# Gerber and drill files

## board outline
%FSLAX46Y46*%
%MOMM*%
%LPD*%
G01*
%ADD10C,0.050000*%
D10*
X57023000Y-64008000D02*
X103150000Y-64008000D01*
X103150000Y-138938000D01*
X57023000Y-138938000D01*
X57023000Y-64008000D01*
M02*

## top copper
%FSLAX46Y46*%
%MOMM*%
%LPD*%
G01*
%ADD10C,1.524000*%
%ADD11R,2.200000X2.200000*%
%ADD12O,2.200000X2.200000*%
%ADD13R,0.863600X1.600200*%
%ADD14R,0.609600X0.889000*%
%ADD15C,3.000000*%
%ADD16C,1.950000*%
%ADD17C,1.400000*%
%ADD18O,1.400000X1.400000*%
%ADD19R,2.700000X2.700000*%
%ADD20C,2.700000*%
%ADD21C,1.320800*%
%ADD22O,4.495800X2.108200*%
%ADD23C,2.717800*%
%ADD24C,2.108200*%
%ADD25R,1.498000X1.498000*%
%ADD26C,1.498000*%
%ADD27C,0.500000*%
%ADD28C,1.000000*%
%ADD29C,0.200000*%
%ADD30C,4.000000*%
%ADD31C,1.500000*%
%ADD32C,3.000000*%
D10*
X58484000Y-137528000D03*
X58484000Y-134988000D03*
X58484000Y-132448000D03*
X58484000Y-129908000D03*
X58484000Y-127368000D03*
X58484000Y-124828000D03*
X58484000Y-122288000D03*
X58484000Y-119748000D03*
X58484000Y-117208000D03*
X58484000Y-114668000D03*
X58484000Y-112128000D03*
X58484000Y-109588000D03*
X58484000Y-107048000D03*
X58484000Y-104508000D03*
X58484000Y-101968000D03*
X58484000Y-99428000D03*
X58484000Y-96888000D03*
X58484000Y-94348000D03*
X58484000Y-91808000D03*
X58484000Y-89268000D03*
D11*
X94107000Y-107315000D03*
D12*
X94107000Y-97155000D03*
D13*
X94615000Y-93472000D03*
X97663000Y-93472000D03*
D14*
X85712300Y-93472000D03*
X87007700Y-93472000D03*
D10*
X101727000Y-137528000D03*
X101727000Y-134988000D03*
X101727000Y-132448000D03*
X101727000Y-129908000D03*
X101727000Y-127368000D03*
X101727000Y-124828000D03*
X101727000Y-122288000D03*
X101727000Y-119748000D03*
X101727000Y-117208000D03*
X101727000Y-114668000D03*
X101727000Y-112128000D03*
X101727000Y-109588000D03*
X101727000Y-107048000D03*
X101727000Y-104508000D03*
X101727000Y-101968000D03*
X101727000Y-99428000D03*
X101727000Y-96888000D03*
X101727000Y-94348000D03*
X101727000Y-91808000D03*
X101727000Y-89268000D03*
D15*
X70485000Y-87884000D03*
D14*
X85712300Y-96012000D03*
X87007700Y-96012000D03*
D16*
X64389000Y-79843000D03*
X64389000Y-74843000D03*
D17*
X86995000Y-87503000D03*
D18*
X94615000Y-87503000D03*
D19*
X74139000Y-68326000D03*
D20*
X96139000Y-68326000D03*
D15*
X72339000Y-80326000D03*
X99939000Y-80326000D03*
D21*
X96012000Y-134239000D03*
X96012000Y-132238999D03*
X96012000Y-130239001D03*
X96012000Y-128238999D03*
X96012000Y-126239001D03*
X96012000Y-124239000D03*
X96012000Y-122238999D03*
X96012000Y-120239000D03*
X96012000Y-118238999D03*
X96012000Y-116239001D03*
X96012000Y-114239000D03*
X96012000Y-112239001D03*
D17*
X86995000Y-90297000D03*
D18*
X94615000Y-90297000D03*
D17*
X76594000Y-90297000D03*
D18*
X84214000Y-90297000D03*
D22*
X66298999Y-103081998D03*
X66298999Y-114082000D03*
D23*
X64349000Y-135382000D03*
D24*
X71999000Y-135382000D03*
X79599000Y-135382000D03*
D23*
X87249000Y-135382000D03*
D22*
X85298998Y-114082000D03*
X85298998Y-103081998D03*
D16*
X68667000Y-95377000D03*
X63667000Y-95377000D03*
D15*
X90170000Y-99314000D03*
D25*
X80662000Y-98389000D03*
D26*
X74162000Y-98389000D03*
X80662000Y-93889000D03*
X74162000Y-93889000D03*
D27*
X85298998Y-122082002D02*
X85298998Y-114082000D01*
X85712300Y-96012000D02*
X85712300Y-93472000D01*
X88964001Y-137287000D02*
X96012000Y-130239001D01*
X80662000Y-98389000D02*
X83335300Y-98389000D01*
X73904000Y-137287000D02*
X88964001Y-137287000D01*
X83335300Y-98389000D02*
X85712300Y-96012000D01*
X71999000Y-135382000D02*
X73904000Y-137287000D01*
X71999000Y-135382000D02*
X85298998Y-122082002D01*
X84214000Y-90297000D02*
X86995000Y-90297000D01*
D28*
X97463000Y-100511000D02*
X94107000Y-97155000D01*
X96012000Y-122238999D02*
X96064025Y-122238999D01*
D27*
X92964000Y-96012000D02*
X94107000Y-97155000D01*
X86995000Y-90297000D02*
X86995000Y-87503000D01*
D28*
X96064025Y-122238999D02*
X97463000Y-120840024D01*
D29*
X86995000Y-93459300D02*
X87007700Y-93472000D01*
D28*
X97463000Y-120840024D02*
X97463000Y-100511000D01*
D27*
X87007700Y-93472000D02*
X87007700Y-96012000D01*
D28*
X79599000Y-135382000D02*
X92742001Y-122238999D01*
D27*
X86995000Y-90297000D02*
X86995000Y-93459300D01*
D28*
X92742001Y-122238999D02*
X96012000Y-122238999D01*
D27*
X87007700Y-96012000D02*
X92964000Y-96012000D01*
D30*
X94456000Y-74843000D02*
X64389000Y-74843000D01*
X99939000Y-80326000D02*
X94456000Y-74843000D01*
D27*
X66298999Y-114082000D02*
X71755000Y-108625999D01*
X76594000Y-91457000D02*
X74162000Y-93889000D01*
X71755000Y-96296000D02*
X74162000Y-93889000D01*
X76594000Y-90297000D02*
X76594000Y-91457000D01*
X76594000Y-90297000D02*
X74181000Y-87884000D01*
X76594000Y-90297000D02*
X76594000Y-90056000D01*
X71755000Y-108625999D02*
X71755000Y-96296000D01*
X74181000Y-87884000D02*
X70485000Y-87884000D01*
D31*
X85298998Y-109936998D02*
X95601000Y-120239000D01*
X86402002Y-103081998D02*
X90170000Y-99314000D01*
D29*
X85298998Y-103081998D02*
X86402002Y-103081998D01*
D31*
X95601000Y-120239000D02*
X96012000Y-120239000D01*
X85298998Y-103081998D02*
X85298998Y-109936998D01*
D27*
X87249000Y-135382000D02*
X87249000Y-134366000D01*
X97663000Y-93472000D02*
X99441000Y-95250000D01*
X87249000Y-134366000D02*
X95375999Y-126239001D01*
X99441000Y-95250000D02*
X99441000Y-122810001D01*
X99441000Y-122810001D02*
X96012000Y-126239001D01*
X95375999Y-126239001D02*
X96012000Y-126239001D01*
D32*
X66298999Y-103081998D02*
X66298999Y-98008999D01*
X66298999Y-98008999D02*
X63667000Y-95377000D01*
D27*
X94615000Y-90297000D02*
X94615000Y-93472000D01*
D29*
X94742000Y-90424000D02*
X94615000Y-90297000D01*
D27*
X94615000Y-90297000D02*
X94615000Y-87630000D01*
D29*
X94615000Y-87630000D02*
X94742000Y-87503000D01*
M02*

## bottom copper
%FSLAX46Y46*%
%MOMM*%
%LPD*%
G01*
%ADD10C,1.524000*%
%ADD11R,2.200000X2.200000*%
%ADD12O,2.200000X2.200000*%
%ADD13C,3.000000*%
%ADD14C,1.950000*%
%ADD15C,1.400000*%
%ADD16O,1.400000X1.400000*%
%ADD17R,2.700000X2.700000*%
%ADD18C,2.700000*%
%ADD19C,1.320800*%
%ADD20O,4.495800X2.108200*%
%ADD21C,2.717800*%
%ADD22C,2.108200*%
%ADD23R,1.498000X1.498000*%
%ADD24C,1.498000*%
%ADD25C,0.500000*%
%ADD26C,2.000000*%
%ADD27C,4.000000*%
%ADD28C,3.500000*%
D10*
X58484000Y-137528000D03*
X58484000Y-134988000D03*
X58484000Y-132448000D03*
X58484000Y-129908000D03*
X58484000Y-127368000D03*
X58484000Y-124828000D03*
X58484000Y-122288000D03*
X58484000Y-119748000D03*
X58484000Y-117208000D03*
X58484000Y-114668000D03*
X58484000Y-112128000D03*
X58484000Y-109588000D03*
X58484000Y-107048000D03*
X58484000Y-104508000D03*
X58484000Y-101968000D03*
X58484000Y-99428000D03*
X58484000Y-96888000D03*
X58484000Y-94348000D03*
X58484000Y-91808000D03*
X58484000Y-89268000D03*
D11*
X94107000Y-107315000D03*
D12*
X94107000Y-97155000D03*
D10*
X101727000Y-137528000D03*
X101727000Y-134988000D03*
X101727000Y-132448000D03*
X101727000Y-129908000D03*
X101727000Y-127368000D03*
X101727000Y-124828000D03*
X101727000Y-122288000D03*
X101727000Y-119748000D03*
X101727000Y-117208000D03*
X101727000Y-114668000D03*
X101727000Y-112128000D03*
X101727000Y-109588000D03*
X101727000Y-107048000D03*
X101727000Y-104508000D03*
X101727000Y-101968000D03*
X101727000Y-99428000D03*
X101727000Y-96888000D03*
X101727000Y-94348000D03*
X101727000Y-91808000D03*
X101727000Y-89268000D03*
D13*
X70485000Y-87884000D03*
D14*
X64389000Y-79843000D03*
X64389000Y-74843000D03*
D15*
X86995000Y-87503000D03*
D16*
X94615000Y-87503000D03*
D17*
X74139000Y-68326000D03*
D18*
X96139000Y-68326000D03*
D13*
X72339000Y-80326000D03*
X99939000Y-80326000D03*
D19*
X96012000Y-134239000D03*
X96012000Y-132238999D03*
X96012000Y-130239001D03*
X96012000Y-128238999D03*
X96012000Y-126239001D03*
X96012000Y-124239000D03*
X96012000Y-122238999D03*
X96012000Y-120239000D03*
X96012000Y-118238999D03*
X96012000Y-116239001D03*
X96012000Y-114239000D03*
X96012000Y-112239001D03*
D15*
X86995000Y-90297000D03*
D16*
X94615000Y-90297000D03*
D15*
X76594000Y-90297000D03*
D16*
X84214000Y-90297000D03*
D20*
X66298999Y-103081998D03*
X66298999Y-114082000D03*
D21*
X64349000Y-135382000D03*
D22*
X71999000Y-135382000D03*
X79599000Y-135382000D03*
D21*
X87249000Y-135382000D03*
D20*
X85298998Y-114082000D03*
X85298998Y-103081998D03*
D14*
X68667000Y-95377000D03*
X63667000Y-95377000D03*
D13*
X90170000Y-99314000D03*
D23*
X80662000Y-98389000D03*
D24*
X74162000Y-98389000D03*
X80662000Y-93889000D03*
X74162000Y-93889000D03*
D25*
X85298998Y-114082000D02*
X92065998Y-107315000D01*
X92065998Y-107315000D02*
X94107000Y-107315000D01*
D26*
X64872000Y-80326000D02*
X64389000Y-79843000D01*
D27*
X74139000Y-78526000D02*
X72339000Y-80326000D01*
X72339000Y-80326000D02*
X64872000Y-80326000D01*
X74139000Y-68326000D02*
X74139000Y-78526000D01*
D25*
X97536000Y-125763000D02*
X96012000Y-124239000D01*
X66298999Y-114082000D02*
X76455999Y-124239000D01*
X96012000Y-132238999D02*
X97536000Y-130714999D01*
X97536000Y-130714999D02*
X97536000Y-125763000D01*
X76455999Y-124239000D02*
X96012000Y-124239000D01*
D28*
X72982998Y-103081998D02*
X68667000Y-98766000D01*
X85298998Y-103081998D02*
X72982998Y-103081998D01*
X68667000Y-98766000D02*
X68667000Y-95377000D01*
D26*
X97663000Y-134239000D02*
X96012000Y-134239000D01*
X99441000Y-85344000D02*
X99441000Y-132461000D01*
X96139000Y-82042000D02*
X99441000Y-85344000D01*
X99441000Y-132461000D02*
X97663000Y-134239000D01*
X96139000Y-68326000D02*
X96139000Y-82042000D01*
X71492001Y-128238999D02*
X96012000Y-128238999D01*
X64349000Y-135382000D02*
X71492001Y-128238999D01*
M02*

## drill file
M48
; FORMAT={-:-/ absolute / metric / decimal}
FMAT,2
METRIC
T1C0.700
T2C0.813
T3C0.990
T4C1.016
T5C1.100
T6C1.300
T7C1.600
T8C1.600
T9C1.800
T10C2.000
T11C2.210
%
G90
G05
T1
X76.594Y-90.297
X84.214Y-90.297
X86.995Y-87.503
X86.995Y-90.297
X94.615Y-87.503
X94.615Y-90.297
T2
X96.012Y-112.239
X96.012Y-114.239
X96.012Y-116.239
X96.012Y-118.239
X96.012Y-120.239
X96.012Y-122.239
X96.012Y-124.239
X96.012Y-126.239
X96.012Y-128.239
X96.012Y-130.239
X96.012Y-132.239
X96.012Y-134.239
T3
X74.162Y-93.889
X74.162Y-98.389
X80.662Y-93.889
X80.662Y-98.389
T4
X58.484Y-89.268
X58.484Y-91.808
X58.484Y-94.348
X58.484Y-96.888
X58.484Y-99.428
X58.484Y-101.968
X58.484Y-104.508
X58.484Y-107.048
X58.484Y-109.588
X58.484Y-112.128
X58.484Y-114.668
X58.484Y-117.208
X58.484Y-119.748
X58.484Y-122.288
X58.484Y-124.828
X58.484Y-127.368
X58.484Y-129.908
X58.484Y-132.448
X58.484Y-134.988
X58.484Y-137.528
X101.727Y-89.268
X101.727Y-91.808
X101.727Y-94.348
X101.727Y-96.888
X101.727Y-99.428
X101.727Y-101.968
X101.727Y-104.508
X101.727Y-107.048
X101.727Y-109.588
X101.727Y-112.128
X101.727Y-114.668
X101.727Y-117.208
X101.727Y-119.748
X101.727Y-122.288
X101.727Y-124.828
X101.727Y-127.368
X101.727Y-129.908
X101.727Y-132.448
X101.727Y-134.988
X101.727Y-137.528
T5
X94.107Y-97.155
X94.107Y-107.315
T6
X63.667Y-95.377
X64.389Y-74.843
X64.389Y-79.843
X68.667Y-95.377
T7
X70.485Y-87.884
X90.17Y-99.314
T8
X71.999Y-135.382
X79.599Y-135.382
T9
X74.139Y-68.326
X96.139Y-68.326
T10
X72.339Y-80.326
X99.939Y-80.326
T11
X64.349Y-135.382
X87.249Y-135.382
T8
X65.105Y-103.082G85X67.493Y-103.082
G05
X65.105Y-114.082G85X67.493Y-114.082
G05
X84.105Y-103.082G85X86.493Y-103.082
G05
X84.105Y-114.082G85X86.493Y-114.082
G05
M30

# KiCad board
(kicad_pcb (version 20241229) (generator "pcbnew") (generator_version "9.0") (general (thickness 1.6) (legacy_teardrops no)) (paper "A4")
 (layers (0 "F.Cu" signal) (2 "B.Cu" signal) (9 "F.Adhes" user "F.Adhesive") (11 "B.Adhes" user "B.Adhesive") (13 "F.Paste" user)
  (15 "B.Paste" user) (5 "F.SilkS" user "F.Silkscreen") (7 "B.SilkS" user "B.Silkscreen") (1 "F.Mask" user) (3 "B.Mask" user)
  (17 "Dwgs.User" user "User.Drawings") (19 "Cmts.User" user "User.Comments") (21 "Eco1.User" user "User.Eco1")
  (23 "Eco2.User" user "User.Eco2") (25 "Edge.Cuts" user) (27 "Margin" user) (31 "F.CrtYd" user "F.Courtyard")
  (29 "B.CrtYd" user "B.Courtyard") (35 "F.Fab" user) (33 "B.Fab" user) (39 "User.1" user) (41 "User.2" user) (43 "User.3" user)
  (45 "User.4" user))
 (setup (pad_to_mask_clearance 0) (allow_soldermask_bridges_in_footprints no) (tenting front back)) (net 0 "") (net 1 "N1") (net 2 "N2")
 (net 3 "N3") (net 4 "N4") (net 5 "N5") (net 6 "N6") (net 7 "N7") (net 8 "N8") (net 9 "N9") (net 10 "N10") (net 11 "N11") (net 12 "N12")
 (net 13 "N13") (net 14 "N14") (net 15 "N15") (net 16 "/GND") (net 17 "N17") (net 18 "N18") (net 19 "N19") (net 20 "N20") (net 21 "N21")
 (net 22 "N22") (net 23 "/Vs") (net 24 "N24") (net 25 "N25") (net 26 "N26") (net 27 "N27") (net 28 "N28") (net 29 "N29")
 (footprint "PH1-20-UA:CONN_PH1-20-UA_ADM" (layer "F.Cu") (at 58.484 137.528 90)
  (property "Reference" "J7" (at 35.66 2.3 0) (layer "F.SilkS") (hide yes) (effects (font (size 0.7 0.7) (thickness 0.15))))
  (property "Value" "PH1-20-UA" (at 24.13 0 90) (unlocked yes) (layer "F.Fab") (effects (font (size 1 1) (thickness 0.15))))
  (pad "1" thru_hole circle (at 0 0 90) (size 1.524 1.524) (drill 1.016) (layers "*.Cu" "*.Mask") (remove_unused_layers no))
  (pad "2" thru_hole circle (at 2.54 0 90) (size 1.524 1.524) (drill 1.016) (layers "*.Cu" "*.Mask") (remove_unused_layers no))
  (pad "3" thru_hole circle (at 5.08 0 90) (size 1.524 1.524) (drill 1.016) (layers "*.Cu" "*.Mask") (remove_unused_layers no))
  (pad "4" thru_hole circle (at 7.62 0 90) (size 1.524 1.524) (drill 1.016) (layers "*.Cu" "*.Mask") (remove_unused_layers no))
  (pad "5" thru_hole circle (at 10.16 0 90) (size 1.524 1.524) (drill 1.016) (layers "*.Cu" "*.Mask") (remove_unused_layers no))
  (pad "6" thru_hole circle (at 12.7 0 90) (size 1.524 1.524) (drill 1.016) (layers "*.Cu" "*.Mask") (remove_unused_layers no))
  (pad "7" thru_hole circle (at 15.24 0 90) (size 1.524 1.524) (drill 1.016) (layers "*.Cu" "*.Mask") (remove_unused_layers no) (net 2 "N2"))
  (pad "8" thru_hole circle (at 17.78 0 90) (size 1.524 1.524) (drill 1.016) (layers "*.Cu" "*.Mask") (remove_unused_layers no) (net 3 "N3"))
  (pad "9" thru_hole circle (at 20.32 0 90) (size 1.524 1.524) (drill 1.016) (layers "*.Cu" "*.Mask") (remove_unused_layers no) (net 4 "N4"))
  (pad "10" thru_hole circle (at 22.86 0 90) (size 1.524 1.524) (drill 1.016) (layers "*.Cu" "*.Mask") (remove_unused_layers no)
   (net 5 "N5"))
  (pad "11" thru_hole circle (at 25.4 0 90) (size 1.524 1.524) (drill 1.016) (layers "*.Cu" "*.Mask") (remove_unused_layers no) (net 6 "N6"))
  (pad "12" thru_hole circle (at 27.94 0 90) (size 1.524 1.524) (drill 1.016) (layers "*.Cu" "*.Mask") (remove_unused_layers no)
   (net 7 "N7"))
  (pad "13" thru_hole circle (at 30.48 0 90) (size 1.524 1.524) (drill 1.016) (layers "*.Cu" "*.Mask") (remove_unused_layers no)
   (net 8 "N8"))
  (pad "14" thru_hole circle (at 33.02 0 90) (size 1.524 1.524) (drill 1.016) (layers "*.Cu" "*.Mask") (remove_unused_layers no)
   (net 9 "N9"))
  (pad "15" thru_hole circle (at 35.56 0 90) (size 1.524 1.524) (drill 1.016) (layers "*.Cu" "*.Mask") (remove_unused_layers no)
   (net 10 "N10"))
  (pad "16" thru_hole circle (at 38.1 0 90) (size 1.524 1.524) (drill 1.016) (layers "*.Cu" "*.Mask") (remove_unused_layers no)
   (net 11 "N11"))
  (pad "17" thru_hole circle (at 40.64 0 90) (size 1.524 1.524) (drill 1.016) (layers "*.Cu" "*.Mask") (remove_unused_layers no)
   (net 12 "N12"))
  (pad "18" thru_hole circle (at 43.18 0 90) (size 1.524 1.524) (drill 1.016) (layers "*.Cu" "*.Mask") (remove_unused_layers no)
   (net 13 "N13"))
  (pad "19" thru_hole circle (at 45.72 0 90) (size 1.524 1.524) (drill 1.016) (layers "*.Cu" "*.Mask") (remove_unused_layers no)
   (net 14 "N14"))
  (pad "20" thru_hole circle (at 48.26 0 90) (size 1.524 1.524) (drill 1.016) (layers "*.Cu" "*.Mask") (remove_unused_layers no)
   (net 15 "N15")))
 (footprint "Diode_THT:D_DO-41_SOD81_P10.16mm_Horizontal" (layer "F.Cu") (at 94.107 107.315 90)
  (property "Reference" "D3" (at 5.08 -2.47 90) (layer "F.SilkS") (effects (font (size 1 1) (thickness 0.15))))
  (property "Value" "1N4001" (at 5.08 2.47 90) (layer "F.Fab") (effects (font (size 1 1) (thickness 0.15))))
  (pad "1" thru_hole rect (at 0 0 90) (size 2.2 2.2) (drill 1.1) (layers "*.Cu" "*.Mask") (remove_unused_layers no) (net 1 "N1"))
  (pad "2" thru_hole oval (at 10.16 0 90) (size 2.2 2.2) (drill 1.1) (layers "*.Cu" "*.Mask") (remove_unused_layers no) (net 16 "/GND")))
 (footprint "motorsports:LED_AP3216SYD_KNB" (layer "F.Cu") (at 96.139 93.472)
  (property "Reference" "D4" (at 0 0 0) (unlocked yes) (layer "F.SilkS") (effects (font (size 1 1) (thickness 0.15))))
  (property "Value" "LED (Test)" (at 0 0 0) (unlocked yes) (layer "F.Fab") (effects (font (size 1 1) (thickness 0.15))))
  (pad "1" smd rect (at -1.524 0) (size 0.8636 1.6002) (layers "F.Cu" "F.Mask" "F.Paste") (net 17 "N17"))
  (pad "2" smd rect (at 1.524 0) (size 0.8636 1.6002) (layers "F.Cu" "F.Mask" "F.Paste") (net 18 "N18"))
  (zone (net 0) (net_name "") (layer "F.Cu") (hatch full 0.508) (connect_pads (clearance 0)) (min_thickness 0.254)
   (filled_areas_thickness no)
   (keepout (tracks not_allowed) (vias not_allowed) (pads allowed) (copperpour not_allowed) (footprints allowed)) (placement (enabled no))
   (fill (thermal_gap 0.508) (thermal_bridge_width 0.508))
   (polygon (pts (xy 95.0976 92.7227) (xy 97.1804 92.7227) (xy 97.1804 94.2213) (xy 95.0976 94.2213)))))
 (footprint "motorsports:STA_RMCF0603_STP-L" (layer "F.Cu") (at 86.36 93.472)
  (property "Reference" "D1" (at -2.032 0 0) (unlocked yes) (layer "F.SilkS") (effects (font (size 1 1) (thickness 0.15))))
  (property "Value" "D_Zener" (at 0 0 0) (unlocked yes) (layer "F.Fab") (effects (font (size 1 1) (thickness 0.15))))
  (pad "1" smd rect (at -0.6477 0) (size 0.6096 0.889) (layers "F.Cu" "F.Mask" "F.Paste") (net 1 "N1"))
  (pad "2" smd rect (at 0.6477 0) (size 0.6096 0.889) (layers "F.Cu" "F.Mask" "F.Paste") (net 16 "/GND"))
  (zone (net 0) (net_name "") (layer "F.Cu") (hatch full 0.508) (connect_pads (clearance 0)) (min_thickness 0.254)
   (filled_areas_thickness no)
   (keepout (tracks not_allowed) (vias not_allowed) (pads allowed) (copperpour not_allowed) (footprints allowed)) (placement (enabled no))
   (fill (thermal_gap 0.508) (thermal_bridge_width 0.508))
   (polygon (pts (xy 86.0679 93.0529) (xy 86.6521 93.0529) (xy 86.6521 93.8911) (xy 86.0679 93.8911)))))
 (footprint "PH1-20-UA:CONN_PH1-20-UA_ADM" (layer "F.Cu") (at 101.727 137.528 90)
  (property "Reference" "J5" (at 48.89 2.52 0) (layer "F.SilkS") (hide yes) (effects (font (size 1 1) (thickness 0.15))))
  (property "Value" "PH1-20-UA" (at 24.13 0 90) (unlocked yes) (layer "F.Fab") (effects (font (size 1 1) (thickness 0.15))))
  (pad "1" thru_hole circle (at 0 0 90) (size 1.524 1.524) (drill 1.016) (layers "*.Cu" "*.Mask") (remove_unused_layers no))
  (pad "2" thru_hole circle (at 2.54 0 90) (size 1.524 1.524) (drill 1.016) (layers "*.Cu" "*.Mask") (remove_unused_layers no))
  (pad "3" thru_hole circle (at 5.08 0 90) (size 1.524 1.524) (drill 1.016) (layers "*.Cu" "*.Mask") (remove_unused_layers no))
  (pad "4" thru_hole circle (at 7.62 0 90) (size 1.524 1.524) (drill 1.016) (layers "*.Cu" "*.Mask") (remove_unused_layers no))
  (pad "5" thru_hole circle (at 10.16 0 90) (size 1.524 1.524) (drill 1.016) (layers "*.Cu" "*.Mask") (remove_unused_layers no))
  (pad "6" thru_hole circle (at 12.7 0 90) (size 1.524 1.524) (drill 1.016) (layers "*.Cu" "*.Mask") (remove_unused_layers no))
  (pad "7" thru_hole circle (at 15.24 0 90) (size 1.524 1.524) (drill 1.016) (layers "*.Cu" "*.Mask") (remove_unused_layers no))
  (pad "8" thru_hole circle (at 17.78 0 90) (size 1.524 1.524) (drill 1.016) (layers "*.Cu" "*.Mask") (remove_unused_layers no))
  (pad "9" thru_hole circle (at 20.32 0 90) (size 1.524 1.524) (drill 1.016) (layers "*.Cu" "*.Mask") (remove_unused_layers no))
  (pad "10" thru_hole circle (at 22.86 0 90) (size 1.524 1.524) (drill 1.016) (layers "*.Cu" "*.Mask") (remove_unused_layers no))
  (pad "11" thru_hole circle (at 25.4 0 90) (size 1.524 1.524) (drill 1.016) (layers "*.Cu" "*.Mask") (remove_unused_layers no))
  (pad "12" thru_hole circle (at 27.94 0 90) (size 1.524 1.524) (drill 1.016) (layers "*.Cu" "*.Mask") (remove_unused_layers no))
  (pad "13" thru_hole circle (at 30.48 0 90) (size 1.524 1.524) (drill 1.016) (layers "*.Cu" "*.Mask") (remove_unused_layers no))
  (pad "14" thru_hole circle (at 33.02 0 90) (size 1.524 1.524) (drill 1.016) (layers "*.Cu" "*.Mask") (remove_unused_layers no))
  (pad "15" thru_hole circle (at 35.56 0 90) (size 1.524 1.524) (drill 1.016) (layers "*.Cu" "*.Mask") (remove_unused_layers no))
  (pad "16" thru_hole circle (at 38.1 0 90) (size 1.524 1.524) (drill 1.016) (layers "*.Cu" "*.Mask") (remove_unused_layers no))
  (pad "17" thru_hole circle (at 40.64 0 90) (size 1.524 1.524) (drill 1.016) (layers "*.Cu" "*.Mask") (remove_unused_layers no))
  (pad "18" thru_hole circle (at 43.18 0 90) (size 1.524 1.524) (drill 1.016) (layers "*.Cu" "*.Mask") (remove_unused_layers no))
  (pad "19" thru_hole circle (at 45.72 0 90) (size 1.524 1.524) (drill 1.016) (layers "*.Cu" "*.Mask") (remove_unused_layers no))
  (pad "20" thru_hole circle (at 48.26 0 90) (size 1.524 1.524) (drill 1.016) (layers "*.Cu" "*.Mask") (remove_unused_layers no)))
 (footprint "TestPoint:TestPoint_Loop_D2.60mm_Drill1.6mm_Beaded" (layer "F.Cu") (at 70.485 87.884)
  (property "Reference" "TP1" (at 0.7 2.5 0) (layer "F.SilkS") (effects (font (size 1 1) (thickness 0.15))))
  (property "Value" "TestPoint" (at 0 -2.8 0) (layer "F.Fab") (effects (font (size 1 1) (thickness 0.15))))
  (pad "1" thru_hole circle (at 0 0) (size 3 3) (drill 1.6) (layers "*.Cu" "*.Mask") (remove_unused_layers no) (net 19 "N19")))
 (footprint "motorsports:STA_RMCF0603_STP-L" (layer "F.Cu") (at 86.36 96.012)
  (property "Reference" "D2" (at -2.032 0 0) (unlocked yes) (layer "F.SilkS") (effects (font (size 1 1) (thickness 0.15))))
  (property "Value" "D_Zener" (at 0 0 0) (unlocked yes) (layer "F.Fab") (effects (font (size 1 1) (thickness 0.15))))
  (pad "1" smd rect (at -0.6477 0) (size 0.6096 0.889) (layers "F.Cu" "F.Mask" "F.Paste") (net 1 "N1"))
  (pad "2" smd rect (at 0.6477 0) (size 0.6096 0.889) (layers "F.Cu" "F.Mask" "F.Paste") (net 16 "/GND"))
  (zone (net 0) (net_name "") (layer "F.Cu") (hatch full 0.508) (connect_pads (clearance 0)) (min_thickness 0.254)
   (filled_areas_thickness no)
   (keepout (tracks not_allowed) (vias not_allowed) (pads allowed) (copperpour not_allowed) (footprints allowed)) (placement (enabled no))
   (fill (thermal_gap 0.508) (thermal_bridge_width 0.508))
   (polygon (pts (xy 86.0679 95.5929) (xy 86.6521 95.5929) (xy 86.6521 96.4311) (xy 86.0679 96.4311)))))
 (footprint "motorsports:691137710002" (layer "F.Cu") (at 64.389 77.343 90)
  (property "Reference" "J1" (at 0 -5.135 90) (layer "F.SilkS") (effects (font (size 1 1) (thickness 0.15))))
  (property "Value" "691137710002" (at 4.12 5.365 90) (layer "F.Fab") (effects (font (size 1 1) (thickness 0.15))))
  (pad "1" thru_hole circle (at -2.5 0 90) (size 1.95 1.95) (drill 1.3) (layers "*.Cu" "*.Mask") (remove_unused_layers no) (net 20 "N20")
   (solder_mask_margin 0.102))
  (pad "2" thru_hole circle (at 2.5 0 90) (size 1.95 1.95) (drill 1.3) (layers "*.Cu" "*.Mask") (remove_unused_layers no) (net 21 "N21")
   (solder_mask_margin 0.102)))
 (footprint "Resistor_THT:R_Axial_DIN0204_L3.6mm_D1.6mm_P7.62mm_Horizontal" (layer "F.Cu") (at 86.995 87.503)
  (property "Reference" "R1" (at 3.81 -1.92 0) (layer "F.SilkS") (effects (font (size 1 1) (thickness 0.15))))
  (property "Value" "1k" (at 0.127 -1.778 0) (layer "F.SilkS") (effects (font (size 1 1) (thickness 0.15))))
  (pad "1" thru_hole circle (at 0 0) (size 1.4 1.4) (drill 0.7) (layers "*.Cu" "*.Mask") (remove_unused_layers no) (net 16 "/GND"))
  (pad "2" thru_hole oval (at 7.62 0) (size 1.4 1.4) (drill 0.7) (layers "*.Cu" "*.Mask") (remove_unused_layers no) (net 17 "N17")))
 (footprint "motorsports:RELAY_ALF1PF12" (layer "F.Cu") (at 86.139 74.326)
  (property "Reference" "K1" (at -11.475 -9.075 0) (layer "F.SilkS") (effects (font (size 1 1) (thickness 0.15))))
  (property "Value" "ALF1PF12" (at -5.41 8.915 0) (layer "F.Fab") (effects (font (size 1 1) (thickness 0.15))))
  (pad "1" thru_hole rect (at -12 -6) (size 2.7 2.7) (drill 1.8) (layers "*.Cu" "*.Mask") (remove_unused_layers no) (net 20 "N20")
   (solder_mask_margin 0.102))
  (pad "2" thru_hole circle (at 10 -6) (size 2.7 2.7) (drill 1.8) (layers "*.Cu" "*.Mask") (remove_unused_layers no) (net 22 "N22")
   (solder_mask_margin 0.102))
  (pad "3" thru_hole circle (at -13.8 6) (size 3 3) (drill 2) (layers "*.Cu" "*.Mask") (remove_unused_layers no) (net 20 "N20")
   (solder_mask_margin 0.102))
  (pad "4" thru_hole circle (at 13.8 6) (size 3 3) (drill 2) (layers "*.Cu" "*.Mask") (remove_unused_layers no) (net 21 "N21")
   (solder_mask_margin 0.102)))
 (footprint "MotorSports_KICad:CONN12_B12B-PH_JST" (layer "F.Cu") (at 96.012 134.239 90)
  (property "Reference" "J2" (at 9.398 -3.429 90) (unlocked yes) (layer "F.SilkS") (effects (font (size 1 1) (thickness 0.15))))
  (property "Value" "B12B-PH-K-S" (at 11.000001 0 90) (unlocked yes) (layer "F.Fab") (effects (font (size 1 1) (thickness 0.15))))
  (pad "1" thru_hole circle (at 0 0 90) (size 1.3208 1.3208) (drill 0.8128) (layers "*.Cu" "*.Mask") (remove_unused_layers no)
   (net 22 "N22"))
  (pad "2" thru_hole circle (at 2.000001 0 90) (size 1.3208 1.3208) (drill 0.8128) (layers "*.Cu" "*.Mask") (remove_unused_layers no)
   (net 19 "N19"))
  (pad "3" thru_hole circle (at 3.999999 0 90) (size 1.3208 1.3208) (drill 0.8128) (layers "*.Cu" "*.Mask") (remove_unused_layers no)
   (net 1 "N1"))
  (pad "4" thru_hole circle (at 6.000001 0 90) (size 1.3208 1.3208) (drill 0.8128) (layers "*.Cu" "*.Mask") (remove_unused_layers no)
   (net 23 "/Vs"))
  (pad "5" thru_hole circle (at 7.999999 0 90) (size 1.3208 1.3208) (drill 0.8128) (layers "*.Cu" "*.Mask") (remove_unused_layers no)
   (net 18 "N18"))
  (pad "6" thru_hole circle (at 10 0 90) (size 1.3208 1.3208) (drill 0.8128) (layers "*.Cu" "*.Mask") (remove_unused_layers no)
   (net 19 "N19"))
  (pad "7" thru_hole circle (at 12.000001 0 90) (size 1.3208 1.3208) (drill 0.8128) (layers "*.Cu" "*.Mask") (remove_unused_layers no)
   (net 16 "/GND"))
  (pad "8" thru_hole circle (at 14 0 90) (size 1.3208 1.3208) (drill 0.8128) (layers "*.Cu" "*.Mask") (remove_unused_layers no)
   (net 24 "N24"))
  (pad "9" thru_hole circle (at 16.000001 0 90) (size 1.3208 1.3208) (drill 0.8128) (layers "*.Cu" "*.Mask") (remove_unused_layers no)
   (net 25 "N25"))
  (pad "10" thru_hole circle (at 17.999999 0 90) (size 1.3208 1.3208) (drill 0.8128) (layers "*.Cu" "*.Mask") (remove_unused_layers no)
   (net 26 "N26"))
  (pad "11" thru_hole circle (at 20 0 90) (size 1.3208 1.3208) (drill 0.8128) (layers "*.Cu" "*.Mask") (remove_unused_layers no)
   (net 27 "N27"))
  (pad "12" thru_hole circle (at 21.999999 0 90) (size 1.3208 1.3208) (drill 0.8128) (layers "*.Cu" "*.Mask") (remove_unused_layers no)
   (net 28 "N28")))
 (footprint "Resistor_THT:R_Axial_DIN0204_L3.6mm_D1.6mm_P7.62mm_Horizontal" (layer "F.Cu") (at 86.995 90.297)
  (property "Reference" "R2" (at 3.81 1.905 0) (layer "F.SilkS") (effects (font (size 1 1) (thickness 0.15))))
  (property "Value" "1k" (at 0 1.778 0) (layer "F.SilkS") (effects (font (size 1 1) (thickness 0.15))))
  (pad "1" thru_hole circle (at 0 0) (size 1.4 1.4) (drill 0.7) (layers "*.Cu" "*.Mask") (remove_unused_layers no) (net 16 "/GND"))
  (pad "2" thru_hole oval (at 7.62 0) (size 1.4 1.4) (drill 0.7) (layers "*.Cu" "*.Mask") (remove_unused_layers no) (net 17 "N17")))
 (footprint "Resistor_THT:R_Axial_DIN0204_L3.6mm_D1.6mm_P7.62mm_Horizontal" (layer "F.Cu") (at 76.594 90.297)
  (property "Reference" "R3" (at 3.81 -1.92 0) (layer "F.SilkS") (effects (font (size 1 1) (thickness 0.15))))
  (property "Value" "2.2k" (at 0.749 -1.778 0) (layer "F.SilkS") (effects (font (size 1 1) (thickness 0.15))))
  (pad "1" thru_hole circle (at 0 0) (size 1.4 1.4) (drill 0.7) (layers "*.Cu" "*.Mask") (remove_unused_layers no) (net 19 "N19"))
  (pad "2" thru_hole oval (at 7.62 0) (size 1.4 1.4) (drill 0.7) (layers "*.Cu" "*.Mask") (remove_unused_layers no) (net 16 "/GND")))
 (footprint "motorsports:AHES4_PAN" (layer "F.Cu") (at 66.298999 103.081998)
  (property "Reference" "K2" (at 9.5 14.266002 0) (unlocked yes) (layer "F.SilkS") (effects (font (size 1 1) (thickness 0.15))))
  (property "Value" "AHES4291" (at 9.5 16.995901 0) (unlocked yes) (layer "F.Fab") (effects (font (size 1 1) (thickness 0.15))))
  (pad "1" thru_hole oval (at 0 0) (size 4.4958 2.1082) (drill oval 3.9878 1.6002) (layers "*.Cu" "*.Mask") (remove_unused_layers no)
   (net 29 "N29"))
  (pad "2" thru_hole oval (at 0 11.000002) (size 4.4958 2.1082) (drill oval 3.9878 1.6002) (layers "*.Cu" "*.Mask")
   (remove_unused_layers no) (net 19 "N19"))
  (pad "3" thru_hole circle (at -1.949999 32.300002) (size 2.7178 2.7178) (drill 2.2098) (layers "*.Cu" "*.Mask") (remove_unused_layers no)
   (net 23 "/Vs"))
  (pad "4" thru_hole circle (at 5.700001 32.300002) (size 2.1082 2.1082) (drill 1.6002) (layers "*.Cu" "*.Mask") (remove_unused_layers no)
   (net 1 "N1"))
  (pad "5" thru_hole circle (at 13.300001 32.300002) (size 2.1082 2.1082) (drill 1.6002) (layers "*.Cu" "*.Mask") (remove_unused_layers no)
   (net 16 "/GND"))
  (pad "6" thru_hole circle (at 20.950001 32.300002) (size 2.7178 2.7178) (drill 2.2098) (layers "*.Cu" "*.Mask") (remove_unused_layers no)
   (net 18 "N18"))
  (pad "7" thru_hole oval (at 18.999999 11.000002) (size 4.4958 2.1082) (drill oval 3.9878 1.6002) (layers "*.Cu" "*.Mask")
   (remove_unused_layers no) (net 1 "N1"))
  (pad "8" thru_hole oval (at 18.999999 0) (size 4.4958 2.1082) (drill oval 3.9878 1.6002) (layers "*.Cu" "*.Mask")
   (remove_unused_layers no) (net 24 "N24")))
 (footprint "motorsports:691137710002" (layer "F.Cu") (at 66.167 95.377 180)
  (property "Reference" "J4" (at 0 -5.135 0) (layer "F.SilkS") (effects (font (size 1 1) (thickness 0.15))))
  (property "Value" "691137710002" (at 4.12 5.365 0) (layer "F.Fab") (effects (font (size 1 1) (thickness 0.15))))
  (pad "1" thru_hole circle (at -2.5 0 180) (size 1.95 1.95) (drill 1.3) (layers "*.Cu" "*.Mask") (remove_unused_layers no) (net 24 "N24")
   (solder_mask_margin 0.102))
  (pad "2" thru_hole circle (at 2.5 0 180) (size 1.95 1.95) (drill 1.3) (layers "*.Cu" "*.Mask") (remove_unused_layers no) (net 29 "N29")
   (solder_mask_margin 0.102)))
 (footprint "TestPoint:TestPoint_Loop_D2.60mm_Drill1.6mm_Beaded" (layer "F.Cu") (at 90.17 99.314)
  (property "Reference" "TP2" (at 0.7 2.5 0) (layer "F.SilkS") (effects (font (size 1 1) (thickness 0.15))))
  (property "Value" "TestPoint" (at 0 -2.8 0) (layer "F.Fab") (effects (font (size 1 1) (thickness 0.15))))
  (pad "1" thru_hole circle (at 0 0) (size 3 3) (drill 1.6) (layers "*.Cu" "*.Mask") (remove_unused_layers no) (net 24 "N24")))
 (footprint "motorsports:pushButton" (layer "F.Cu") (at 77.412 96.139 180)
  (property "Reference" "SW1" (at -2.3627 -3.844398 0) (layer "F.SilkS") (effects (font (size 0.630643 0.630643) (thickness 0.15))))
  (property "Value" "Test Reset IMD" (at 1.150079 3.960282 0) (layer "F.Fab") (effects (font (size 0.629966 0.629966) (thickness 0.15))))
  (pad "1" thru_hole rect (at -3.25 -2.25 180) (size 1.498 1.498) (drill 0.99) (layers "*.Cu" "*.Mask") (remove_unused_layers no)
   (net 1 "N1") (solder_mask_margin 0.102))
  (pad "2" thru_hole circle (at 3.25 -2.25 180) (size 1.498 1.498) (drill 0.99) (layers "*.Cu" "*.Mask") (remove_unused_layers no)
   (solder_mask_margin 0.102))
  (pad "3" thru_hole circle (at -3.25 2.25 180) (size 1.498 1.498) (drill 0.99) (layers "*.Cu" "*.Mask") (remove_unused_layers no)
   (solder_mask_margin 0.102))
  (pad "4" thru_hole circle (at 3.25 2.25 180) (size 1.498 1.498) (drill 0.99) (layers "*.Cu" "*.Mask") (remove_unused_layers no)
   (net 19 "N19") (solder_mask_margin 0.102)))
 (gr_rect (start 57.023 64.008) (end 103.15 138.938) (stroke (width 0.05) (type default)) (fill no) (layer "Edge.Cuts"))
 (segment (start 85.298998 122.082002) (end 85.298998 114.082) (width 0.5) (layer "F.Cu") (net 1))
 (segment (start 85.7123 96.012) (end 85.7123 93.472) (width 0.5) (layer "F.Cu") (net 1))
 (segment (start 88.964001 137.287) (end 96.012 130.239001) (width 0.5) (layer "F.Cu") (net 1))
 (segment (start 80.662 98.389) (end 83.3353 98.389) (width 0.5) (layer "F.Cu") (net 1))
 (segment (start 73.904 137.287) (end 88.964001 137.287) (width 0.5) (layer "F.Cu") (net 1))
 (segment (start 83.3353 98.389) (end 85.7123 96.012) (width 0.5) (layer "F.Cu") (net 1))
 (segment (start 71.999 135.382) (end 73.904 137.287) (width 0.5) (layer "F.Cu") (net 1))
 (segment (start 71.999 135.382) (end 85.298998 122.082002) (width 0.5) (layer "F.Cu") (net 1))
 (segment (start 85.298998 114.082) (end 92.065998 107.315) (width 0.5) (layer "B.Cu") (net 1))
 (segment (start 92.065998 107.315) (end 94.107 107.315) (width 0.5) (layer "B.Cu") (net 1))
 (segment (start 84.214 90.297) (end 86.995 90.297) (width 0.5) (layer "F.Cu") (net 16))
 (segment (start 97.463 100.511) (end 94.107 97.155) (width 1) (layer "F.Cu") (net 16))
 (segment (start 96.012 122.238999) (end 96.064025 122.238999) (width 1) (layer "F.Cu") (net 16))
 (segment (start 92.964 96.012) (end 94.107 97.155) (width 0.5) (layer "F.Cu") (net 16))
 (segment (start 86.995 90.297) (end 86.995 87.503) (width 0.5) (layer "F.Cu") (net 16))
 (segment (start 96.064025 122.238999) (end 97.463 120.840024) (width 1) (layer "F.Cu") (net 16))
 (segment (start 86.995 93.4593) (end 87.0077 93.472) (width 0.2) (layer "F.Cu") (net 16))
 (segment (start 97.463 120.840024) (end 97.463 100.511) (width 1) (layer "F.Cu") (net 16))
 (segment (start 87.0077 93.472) (end 87.0077 96.012) (width 0.5) (layer "F.Cu") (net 16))
 (segment (start 79.599 135.382) (end 92.742001 122.238999) (width 1) (layer "F.Cu") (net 16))
 (segment (start 86.995 90.297) (end 86.995 93.4593) (width 0.5) (layer "F.Cu") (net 16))
 (segment (start 92.742001 122.238999) (end 96.012 122.238999) (width 1) (layer "F.Cu") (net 16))
 (segment (start 87.0077 96.012) (end 92.964 96.012) (width 0.5) (layer "F.Cu") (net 16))
 (segment (start 64.872 80.326) (end 64.389 79.843) (width 2) (layer "B.Cu") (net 20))
 (segment (start 74.139 78.526) (end 72.339 80.326) (width 4) (layer "B.Cu") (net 20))
 (segment (start 72.339 80.326) (end 64.872 80.326) (width 4) (layer "B.Cu") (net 20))
 (segment (start 74.139 68.326) (end 74.139 78.526) (width 4) (layer "B.Cu") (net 20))
 (segment (start 94.456 74.843) (end 64.389 74.843) (width 4) (layer "F.Cu") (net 21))
 (segment (start 99.939 80.326) (end 94.456 74.843) (width 4) (layer "F.Cu") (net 21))
 (segment (start 66.298999 114.082) (end 71.755 108.625999) (width 0.5) (layer "F.Cu") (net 19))
 (segment (start 76.594 91.457) (end 74.162 93.889) (width 0.5) (layer "F.Cu") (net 19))
 (segment (start 71.755 96.296) (end 74.162 93.889) (width 0.5) (layer "F.Cu") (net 19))
 (segment (start 76.594 90.297) (end 76.594 91.457) (width 0.5) (layer "F.Cu") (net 19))
 (segment (start 76.594 90.297) (end 74.181 87.884) (width 0.5) (layer "F.Cu") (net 19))
 (segment (start 76.594 90.297) (end 76.594 90.056) (width 0.5) (layer "F.Cu") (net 19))
 (segment (start 71.755 108.625999) (end 71.755 96.296) (width 0.5) (layer "F.Cu") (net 19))
 (segment (start 74.181 87.884) (end 70.485 87.884) (width 0.5) (layer "F.Cu") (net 19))
 (segment (start 97.536 125.763) (end 96.012 124.239) (width 0.5) (layer "B.Cu") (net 19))
 (segment (start 66.298999 114.082) (end 76.455999 124.239) (width 0.5) (layer "B.Cu") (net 19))
 (segment (start 96.012 132.238999) (end 97.536 130.714999) (width 0.5) (layer "B.Cu") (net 19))
 (segment (start 97.536 130.714999) (end 97.536 125.763) (width 0.5) (layer "B.Cu") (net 19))
 (segment (start 76.455999 124.239) (end 96.012 124.239) (width 0.5) (layer "B.Cu") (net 19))
 (segment (start 85.298998 109.936998) (end 95.601 120.239) (width 1.5) (layer "F.Cu") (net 24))
 (segment (start 86.402002 103.081998) (end 90.17 99.314) (width 1.5) (layer "F.Cu") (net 24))
 (segment (start 85.298998 103.081998) (end 86.402002 103.081998) (width 0.2) (layer "F.Cu") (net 24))
 (segment (start 95.601 120.239) (end 96.012 120.239) (width 1.5) (layer "F.Cu") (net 24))
 (segment (start 85.298998 103.081998) (end 85.298998 109.936998) (width 1.5) (layer "F.Cu") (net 24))
 (segment (start 72.982998 103.081998) (end 68.667 98.766) (width 3.5) (layer "B.Cu") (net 24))
 (segment (start 85.298998 103.081998) (end 72.982998 103.081998) (width 3.5) (layer "B.Cu") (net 24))
 (segment (start 68.667 98.766) (end 68.667 95.377) (width 3.5) (layer "B.Cu") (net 24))
 (segment (start 87.249 135.382) (end 87.249 134.366) (width 0.5) (layer "F.Cu") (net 18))
 (segment (start 97.663 93.472) (end 99.441 95.25) (width 0.5) (layer "F.Cu") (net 18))
 (segment (start 87.249 134.366) (end 95.375999 126.239001) (width 0.5) (layer "F.Cu") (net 18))
 (segment (start 99.441 95.25) (end 99.441 122.810001) (width 0.5) (layer "F.Cu") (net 18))
 (segment (start 99.441 122.810001) (end 96.012 126.239001) (width 0.5) (layer "F.Cu") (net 18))
 (segment (start 95.375999 126.239001) (end 96.012 126.239001) (width 0.5) (layer "F.Cu") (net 18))
 (segment (start 97.663 134.239) (end 96.012 134.239) (width 2) (layer "B.Cu") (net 22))
 (segment (start 99.441 85.344) (end 99.441 132.461) (width 2) (layer "B.Cu") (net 22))
 (segment (start 96.139 82.042) (end 99.441 85.344) (width 2) (layer "B.Cu") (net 22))
 (segment (start 99.441 132.461) (end 97.663 134.239) (width 2) (layer "B.Cu") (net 22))
 (segment (start 96.139 68.326) (end 96.139 82.042) (width 2) (layer "B.Cu") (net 22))
 (segment (start 71.492001 128.238999) (end 96.012 128.238999) (width 2) (layer "B.Cu") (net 23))
 (segment (start 64.349 135.382) (end 71.492001 128.238999) (width 2) (layer "B.Cu") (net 23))
 (segment (start 66.298999 103.081998) (end 66.298999 98.008999) (width 3) (layer "F.Cu") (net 29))
 (segment (start 66.298999 98.008999) (end 63.667 95.377) (width 3) (layer "F.Cu") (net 29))
 (segment (start 94.615 90.297) (end 94.615 93.472) (width 0.5) (layer "F.Cu") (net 17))
 (segment (start 94.742 90.424) (end 94.615 90.297) (width 0.2) (layer "F.Cu") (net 17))
 (segment (start 94.615 90.297) (end 94.615 87.63) (width 0.5) (layer "F.Cu") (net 17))
 (segment (start 94.615 87.63) (end 94.742 87.503) (width 0.2) (layer "F.Cu") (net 17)))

